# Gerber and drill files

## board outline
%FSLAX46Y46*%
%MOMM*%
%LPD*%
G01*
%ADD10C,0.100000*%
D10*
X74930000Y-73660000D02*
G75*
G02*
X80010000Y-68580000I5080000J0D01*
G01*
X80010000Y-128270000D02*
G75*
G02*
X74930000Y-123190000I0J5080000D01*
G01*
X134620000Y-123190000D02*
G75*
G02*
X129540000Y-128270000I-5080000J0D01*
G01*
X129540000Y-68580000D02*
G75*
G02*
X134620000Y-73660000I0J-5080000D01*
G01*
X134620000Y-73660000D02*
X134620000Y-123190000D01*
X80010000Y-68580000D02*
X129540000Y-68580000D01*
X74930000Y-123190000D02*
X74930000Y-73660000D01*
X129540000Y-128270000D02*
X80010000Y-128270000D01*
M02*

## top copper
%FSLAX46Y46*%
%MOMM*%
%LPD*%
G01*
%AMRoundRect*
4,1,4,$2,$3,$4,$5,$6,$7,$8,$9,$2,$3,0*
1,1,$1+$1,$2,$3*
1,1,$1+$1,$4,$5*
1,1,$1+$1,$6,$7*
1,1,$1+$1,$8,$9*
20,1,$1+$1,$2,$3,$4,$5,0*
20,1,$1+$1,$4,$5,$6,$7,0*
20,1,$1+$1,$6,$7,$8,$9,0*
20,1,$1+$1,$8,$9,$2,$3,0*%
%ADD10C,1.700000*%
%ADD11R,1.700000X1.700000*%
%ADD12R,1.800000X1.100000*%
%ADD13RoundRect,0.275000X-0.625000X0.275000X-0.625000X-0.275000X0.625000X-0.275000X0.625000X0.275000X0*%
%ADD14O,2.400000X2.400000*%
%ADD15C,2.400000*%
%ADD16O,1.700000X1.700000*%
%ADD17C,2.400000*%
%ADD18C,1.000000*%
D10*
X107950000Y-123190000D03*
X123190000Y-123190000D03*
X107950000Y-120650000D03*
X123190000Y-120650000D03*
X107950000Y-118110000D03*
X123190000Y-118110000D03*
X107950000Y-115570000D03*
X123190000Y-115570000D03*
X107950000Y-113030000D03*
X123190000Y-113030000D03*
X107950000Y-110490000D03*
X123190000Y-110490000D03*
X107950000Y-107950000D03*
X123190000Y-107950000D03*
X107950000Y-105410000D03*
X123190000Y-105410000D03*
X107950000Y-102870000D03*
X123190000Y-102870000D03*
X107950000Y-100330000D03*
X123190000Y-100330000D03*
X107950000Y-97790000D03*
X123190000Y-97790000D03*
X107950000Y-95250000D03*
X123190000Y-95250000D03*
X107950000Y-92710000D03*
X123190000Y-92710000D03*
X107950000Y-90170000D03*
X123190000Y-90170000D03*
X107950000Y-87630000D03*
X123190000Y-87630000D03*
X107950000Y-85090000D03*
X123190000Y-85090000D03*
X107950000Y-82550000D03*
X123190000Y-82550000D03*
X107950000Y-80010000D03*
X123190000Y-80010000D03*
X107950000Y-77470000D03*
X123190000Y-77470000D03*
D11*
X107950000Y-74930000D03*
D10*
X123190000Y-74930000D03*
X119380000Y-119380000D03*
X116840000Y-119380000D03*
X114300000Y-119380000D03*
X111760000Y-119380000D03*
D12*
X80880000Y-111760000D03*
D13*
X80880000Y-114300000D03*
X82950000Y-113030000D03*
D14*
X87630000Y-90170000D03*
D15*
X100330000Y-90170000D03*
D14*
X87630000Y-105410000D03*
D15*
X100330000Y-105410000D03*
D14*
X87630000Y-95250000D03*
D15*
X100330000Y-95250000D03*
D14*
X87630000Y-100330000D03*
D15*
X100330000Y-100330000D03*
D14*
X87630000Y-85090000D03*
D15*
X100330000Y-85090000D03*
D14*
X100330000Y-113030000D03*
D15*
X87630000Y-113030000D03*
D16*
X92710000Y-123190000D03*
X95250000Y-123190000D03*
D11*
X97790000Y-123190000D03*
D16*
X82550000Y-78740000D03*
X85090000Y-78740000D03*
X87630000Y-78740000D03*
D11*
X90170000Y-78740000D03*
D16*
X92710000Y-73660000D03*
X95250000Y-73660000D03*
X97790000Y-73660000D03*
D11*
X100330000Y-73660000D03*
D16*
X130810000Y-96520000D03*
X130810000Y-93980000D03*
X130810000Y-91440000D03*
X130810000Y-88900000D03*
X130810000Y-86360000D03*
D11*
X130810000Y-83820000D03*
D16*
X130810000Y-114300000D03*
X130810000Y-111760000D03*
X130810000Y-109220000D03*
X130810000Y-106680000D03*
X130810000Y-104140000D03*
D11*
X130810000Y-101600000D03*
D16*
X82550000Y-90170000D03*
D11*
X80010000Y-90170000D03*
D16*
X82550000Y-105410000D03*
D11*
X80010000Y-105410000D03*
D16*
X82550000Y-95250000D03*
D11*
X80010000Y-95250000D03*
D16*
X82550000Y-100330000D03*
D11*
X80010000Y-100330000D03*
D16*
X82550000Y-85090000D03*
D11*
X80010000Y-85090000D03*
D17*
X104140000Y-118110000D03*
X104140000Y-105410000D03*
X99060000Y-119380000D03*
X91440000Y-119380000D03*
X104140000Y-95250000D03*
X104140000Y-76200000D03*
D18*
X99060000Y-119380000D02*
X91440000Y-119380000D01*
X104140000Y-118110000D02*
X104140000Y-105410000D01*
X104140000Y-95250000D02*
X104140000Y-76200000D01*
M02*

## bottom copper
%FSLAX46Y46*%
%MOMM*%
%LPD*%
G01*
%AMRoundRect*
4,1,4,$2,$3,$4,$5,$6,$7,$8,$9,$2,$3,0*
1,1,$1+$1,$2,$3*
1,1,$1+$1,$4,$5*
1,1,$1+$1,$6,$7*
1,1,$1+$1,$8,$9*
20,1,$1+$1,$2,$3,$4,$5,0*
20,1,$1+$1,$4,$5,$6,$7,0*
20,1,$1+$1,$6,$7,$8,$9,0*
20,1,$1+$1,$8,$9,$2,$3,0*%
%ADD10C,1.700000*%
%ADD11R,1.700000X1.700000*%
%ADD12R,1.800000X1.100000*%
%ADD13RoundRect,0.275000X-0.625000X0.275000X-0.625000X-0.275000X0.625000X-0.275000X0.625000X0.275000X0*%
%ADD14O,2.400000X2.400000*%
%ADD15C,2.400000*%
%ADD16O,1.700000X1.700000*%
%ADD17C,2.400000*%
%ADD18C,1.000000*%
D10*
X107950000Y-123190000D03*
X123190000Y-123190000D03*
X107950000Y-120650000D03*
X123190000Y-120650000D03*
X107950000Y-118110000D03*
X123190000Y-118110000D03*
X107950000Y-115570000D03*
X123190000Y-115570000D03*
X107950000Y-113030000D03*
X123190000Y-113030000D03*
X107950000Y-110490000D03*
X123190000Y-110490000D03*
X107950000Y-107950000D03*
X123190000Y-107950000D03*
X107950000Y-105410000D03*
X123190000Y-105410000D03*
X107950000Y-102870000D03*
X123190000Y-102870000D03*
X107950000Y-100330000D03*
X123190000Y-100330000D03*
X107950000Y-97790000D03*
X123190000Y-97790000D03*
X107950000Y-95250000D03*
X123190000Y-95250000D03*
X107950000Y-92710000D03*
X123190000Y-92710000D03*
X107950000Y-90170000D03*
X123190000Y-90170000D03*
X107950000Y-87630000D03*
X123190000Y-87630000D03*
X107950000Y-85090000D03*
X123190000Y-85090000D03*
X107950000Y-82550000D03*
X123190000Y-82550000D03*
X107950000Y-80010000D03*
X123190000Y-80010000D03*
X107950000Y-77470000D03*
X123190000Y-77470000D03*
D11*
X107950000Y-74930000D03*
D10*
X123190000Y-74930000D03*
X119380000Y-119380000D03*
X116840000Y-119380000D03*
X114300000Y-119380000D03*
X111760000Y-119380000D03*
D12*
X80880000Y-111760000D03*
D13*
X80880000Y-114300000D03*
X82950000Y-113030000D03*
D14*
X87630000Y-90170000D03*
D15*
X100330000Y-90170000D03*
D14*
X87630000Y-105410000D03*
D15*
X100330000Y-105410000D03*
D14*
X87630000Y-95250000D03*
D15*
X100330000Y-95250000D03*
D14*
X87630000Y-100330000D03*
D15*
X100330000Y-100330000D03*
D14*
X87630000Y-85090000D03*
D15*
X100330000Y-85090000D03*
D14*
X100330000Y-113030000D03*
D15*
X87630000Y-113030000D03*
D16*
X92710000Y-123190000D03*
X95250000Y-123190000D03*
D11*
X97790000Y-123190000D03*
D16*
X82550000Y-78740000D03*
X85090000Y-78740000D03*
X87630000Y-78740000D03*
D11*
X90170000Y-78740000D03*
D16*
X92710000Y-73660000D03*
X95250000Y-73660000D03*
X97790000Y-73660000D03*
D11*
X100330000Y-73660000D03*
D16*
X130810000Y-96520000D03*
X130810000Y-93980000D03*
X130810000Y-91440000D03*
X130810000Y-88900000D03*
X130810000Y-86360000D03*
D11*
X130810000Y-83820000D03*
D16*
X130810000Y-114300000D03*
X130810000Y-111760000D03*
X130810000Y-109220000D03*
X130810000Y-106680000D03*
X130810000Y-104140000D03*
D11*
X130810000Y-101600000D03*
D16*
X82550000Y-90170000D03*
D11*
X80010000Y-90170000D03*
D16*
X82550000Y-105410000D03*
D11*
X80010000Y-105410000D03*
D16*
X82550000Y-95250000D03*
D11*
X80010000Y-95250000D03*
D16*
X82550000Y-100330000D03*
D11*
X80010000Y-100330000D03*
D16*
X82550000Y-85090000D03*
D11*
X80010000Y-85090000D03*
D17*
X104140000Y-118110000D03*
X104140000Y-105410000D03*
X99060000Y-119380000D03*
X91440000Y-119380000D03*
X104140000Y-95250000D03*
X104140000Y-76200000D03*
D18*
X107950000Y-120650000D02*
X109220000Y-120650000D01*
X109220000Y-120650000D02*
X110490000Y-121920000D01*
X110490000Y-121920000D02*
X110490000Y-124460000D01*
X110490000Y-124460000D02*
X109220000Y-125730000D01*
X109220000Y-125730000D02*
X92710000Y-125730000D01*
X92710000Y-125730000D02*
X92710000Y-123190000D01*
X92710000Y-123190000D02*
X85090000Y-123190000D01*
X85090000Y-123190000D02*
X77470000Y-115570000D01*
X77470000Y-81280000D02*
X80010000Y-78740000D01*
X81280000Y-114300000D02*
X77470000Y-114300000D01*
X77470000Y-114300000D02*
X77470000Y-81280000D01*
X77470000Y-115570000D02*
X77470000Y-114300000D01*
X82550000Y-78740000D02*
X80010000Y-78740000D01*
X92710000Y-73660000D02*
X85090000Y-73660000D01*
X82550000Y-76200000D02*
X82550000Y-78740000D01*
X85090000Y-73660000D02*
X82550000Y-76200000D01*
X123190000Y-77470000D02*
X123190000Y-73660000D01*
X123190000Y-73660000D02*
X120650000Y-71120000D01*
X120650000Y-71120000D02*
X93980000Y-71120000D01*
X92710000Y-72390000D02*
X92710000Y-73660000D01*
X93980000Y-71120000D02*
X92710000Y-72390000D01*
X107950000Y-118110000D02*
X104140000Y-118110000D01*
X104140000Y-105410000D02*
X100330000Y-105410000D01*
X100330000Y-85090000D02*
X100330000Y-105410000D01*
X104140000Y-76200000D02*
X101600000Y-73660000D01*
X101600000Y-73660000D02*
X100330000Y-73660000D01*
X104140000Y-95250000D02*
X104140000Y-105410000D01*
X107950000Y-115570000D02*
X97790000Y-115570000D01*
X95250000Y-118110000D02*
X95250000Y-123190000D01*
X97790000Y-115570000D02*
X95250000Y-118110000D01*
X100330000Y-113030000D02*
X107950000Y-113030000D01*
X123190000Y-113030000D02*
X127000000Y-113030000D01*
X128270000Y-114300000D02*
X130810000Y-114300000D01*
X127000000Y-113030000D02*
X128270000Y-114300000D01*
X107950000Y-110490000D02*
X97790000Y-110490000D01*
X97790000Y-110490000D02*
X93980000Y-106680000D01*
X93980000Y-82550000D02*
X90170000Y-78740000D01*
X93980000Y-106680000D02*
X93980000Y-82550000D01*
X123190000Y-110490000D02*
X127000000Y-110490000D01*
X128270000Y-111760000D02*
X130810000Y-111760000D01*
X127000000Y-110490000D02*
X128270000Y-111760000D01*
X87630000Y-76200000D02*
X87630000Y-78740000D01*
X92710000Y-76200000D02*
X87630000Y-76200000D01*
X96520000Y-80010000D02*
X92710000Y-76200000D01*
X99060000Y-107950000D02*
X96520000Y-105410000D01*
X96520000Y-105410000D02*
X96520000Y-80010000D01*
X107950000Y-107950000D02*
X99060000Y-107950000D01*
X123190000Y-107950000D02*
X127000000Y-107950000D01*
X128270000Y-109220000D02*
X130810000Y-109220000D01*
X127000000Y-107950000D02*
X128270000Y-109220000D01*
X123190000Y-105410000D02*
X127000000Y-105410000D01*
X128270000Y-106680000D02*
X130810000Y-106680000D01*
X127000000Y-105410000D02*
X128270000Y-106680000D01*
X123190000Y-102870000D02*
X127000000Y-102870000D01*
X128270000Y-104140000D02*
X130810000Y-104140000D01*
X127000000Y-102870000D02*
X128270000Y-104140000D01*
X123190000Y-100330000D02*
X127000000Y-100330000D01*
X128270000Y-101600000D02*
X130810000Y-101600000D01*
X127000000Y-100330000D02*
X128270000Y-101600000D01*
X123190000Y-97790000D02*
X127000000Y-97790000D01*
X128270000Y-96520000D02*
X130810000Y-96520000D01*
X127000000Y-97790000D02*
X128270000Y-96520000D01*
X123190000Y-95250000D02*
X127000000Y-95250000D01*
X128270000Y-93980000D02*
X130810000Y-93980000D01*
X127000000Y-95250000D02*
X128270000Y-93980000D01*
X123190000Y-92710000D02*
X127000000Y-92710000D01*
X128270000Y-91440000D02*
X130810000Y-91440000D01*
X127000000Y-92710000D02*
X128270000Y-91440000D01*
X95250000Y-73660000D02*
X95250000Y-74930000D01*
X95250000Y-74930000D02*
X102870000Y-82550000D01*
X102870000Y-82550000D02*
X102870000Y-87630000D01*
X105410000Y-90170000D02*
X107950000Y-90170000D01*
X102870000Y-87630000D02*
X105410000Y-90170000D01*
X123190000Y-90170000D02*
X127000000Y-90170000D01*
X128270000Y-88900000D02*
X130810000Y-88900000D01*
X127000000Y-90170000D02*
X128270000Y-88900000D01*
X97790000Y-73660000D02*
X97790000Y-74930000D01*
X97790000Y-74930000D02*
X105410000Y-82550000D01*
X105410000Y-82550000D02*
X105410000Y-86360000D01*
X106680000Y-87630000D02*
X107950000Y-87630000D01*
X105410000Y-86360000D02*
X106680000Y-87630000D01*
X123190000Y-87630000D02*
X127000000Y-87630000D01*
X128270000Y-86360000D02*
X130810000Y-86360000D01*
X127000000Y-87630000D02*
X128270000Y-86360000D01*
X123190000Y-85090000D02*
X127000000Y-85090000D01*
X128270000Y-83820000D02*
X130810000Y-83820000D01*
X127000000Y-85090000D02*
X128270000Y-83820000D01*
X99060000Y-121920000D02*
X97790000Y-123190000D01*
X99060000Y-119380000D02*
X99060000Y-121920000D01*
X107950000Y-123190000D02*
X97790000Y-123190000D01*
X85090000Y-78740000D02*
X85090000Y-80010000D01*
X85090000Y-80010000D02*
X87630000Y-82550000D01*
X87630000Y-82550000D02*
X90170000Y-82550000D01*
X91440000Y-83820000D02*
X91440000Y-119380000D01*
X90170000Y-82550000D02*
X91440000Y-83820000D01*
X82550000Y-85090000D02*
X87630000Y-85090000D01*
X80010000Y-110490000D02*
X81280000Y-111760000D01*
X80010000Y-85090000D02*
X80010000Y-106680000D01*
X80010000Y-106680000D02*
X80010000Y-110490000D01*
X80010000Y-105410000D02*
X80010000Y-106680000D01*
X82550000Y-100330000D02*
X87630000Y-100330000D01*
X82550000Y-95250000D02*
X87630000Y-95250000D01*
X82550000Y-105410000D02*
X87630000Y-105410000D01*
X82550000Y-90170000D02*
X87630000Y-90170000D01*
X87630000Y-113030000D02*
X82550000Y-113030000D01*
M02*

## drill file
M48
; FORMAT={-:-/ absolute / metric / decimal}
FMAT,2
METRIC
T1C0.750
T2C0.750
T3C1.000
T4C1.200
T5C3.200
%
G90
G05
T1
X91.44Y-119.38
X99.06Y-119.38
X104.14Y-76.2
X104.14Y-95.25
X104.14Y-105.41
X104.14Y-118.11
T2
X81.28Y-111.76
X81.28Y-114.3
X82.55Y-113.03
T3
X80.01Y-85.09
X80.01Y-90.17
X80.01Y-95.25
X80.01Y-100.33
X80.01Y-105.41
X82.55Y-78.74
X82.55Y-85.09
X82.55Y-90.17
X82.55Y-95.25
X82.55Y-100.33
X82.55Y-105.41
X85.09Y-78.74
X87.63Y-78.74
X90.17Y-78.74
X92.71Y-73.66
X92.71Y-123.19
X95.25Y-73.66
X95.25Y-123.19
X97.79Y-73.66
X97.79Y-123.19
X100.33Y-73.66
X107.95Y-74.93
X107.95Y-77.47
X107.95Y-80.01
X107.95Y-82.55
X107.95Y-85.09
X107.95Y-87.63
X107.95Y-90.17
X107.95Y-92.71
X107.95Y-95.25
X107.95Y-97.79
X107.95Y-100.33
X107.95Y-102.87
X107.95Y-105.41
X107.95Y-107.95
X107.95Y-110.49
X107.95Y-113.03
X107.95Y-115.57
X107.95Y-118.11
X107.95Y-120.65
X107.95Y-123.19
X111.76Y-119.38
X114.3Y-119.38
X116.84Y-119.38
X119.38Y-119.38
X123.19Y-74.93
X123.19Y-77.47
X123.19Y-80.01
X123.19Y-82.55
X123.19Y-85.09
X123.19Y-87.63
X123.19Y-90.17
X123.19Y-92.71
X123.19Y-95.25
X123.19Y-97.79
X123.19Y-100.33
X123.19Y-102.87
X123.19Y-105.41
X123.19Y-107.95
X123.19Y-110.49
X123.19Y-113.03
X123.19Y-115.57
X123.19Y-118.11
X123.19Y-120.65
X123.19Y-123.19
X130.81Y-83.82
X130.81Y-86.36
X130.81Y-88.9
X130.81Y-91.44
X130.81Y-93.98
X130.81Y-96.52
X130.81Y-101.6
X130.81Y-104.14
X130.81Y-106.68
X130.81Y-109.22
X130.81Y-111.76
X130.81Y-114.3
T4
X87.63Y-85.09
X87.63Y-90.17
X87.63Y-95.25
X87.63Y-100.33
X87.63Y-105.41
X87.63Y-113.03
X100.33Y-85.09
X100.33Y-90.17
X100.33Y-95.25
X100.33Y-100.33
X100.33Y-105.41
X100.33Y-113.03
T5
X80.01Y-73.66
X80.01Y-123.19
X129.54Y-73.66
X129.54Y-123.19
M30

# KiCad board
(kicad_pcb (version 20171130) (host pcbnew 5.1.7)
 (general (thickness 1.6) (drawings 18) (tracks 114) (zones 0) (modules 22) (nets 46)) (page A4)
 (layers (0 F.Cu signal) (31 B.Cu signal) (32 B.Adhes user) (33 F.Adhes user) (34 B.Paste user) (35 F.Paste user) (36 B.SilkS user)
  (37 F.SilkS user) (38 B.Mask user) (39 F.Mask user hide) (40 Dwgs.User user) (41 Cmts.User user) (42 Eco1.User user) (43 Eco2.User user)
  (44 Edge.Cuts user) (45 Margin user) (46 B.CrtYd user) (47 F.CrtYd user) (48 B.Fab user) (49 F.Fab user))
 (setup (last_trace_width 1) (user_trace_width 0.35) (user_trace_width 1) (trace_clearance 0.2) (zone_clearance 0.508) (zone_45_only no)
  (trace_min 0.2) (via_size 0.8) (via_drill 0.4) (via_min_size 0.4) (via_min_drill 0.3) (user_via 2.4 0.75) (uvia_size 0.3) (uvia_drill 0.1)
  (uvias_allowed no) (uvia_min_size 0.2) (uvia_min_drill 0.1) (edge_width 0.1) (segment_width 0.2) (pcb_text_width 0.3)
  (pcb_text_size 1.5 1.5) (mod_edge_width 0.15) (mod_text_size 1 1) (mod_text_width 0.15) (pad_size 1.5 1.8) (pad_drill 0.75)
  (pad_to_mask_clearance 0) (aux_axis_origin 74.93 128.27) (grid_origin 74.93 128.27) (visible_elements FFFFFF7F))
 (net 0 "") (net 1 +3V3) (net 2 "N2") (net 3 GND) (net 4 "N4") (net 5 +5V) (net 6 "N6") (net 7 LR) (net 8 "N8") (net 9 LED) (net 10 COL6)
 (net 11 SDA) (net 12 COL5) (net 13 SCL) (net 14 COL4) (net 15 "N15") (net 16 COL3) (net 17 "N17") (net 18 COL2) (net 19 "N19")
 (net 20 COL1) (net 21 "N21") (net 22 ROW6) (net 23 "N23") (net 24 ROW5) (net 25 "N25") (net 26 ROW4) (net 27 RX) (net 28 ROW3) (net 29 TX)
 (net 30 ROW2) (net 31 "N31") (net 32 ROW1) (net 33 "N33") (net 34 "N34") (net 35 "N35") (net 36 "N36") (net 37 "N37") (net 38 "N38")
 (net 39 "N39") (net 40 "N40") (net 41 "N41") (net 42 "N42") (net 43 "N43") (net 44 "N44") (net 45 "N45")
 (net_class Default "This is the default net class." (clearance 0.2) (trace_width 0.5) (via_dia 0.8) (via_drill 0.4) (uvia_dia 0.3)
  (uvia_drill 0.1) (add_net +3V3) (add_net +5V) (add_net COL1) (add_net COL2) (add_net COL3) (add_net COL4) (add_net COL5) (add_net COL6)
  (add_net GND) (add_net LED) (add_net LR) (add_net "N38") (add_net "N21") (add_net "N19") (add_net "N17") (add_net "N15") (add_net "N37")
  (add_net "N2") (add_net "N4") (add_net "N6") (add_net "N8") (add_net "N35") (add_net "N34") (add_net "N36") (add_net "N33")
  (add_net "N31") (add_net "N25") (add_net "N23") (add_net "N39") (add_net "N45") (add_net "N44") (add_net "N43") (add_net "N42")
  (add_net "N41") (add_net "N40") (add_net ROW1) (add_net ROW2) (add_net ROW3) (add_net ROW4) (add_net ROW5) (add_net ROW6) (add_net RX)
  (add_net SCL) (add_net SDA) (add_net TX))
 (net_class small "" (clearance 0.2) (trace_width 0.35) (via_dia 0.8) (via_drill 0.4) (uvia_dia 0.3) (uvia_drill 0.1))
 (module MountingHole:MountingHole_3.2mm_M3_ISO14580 (layer F.Cu) (at 80.01 123.19)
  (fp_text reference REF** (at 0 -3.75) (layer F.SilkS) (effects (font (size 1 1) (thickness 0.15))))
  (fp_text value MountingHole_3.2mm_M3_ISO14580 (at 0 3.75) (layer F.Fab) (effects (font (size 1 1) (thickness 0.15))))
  (pad 1 np_thru_hole circle (at 0 0) (size 3.2 3.2) (drill 3.2) (layers *.Cu *.Mask)))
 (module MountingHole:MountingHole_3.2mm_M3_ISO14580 (layer F.Cu) (at 129.54 123.19)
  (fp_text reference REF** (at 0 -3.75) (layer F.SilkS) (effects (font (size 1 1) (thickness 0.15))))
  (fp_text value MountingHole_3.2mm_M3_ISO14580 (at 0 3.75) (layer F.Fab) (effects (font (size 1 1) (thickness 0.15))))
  (pad 1 np_thru_hole circle (at 0 0) (size 3.2 3.2) (drill 3.2) (layers *.Cu *.Mask)))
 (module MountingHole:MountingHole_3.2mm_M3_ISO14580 (layer F.Cu) (at 129.54 73.66)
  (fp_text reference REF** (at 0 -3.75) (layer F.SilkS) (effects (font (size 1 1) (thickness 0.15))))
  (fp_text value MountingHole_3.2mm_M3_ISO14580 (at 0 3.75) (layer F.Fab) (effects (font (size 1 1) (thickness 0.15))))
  (pad 1 np_thru_hole circle (at 0 0) (size 3.2 3.2) (drill 3.2) (layers *.Cu *.Mask)))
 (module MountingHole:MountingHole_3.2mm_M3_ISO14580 (layer F.Cu) (at 80.01 73.66)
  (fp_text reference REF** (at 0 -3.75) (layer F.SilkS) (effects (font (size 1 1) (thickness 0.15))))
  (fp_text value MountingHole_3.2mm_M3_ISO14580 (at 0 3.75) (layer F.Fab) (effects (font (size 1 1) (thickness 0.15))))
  (pad 1 np_thru_hole circle (at 0 0) (size 3.2 3.2) (drill 3.2) (layers *.Cu *.Mask)))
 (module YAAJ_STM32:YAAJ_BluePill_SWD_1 (layer F.Cu) (at 107.95 74.93)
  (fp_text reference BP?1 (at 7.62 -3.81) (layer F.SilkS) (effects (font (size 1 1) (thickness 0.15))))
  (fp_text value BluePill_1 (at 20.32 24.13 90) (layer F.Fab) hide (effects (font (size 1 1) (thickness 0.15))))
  (pad 20 thru_hole circle (at 0 48.26) (size 1.7 1.7) (drill 1) (layers *.Cu *.Mask) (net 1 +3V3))
  (pad 21 thru_hole circle (at 15.24 48.26) (size 1.7 1.7) (drill 1) (layers *.Cu *.Mask) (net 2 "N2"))
  (pad 19 thru_hole circle (at 0 45.72) (size 1.7 1.7) (drill 1) (layers *.Cu *.Mask) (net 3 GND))
  (pad 22 thru_hole circle (at 15.24 45.72) (size 1.7 1.7) (drill 1) (layers *.Cu *.Mask) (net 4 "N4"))
  (pad 18 thru_hole circle (at 0 43.18) (size 1.7 1.7) (drill 1) (layers *.Cu *.Mask) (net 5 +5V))
  (pad 23 thru_hole circle (at 15.24 43.18) (size 1.7 1.7) (drill 1) (layers *.Cu *.Mask) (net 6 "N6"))
  (pad 17 thru_hole circle (at 0 40.64) (size 1.7 1.7) (drill 1) (layers *.Cu *.Mask) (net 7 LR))
  (pad 24 thru_hole circle (at 15.24 40.64) (size 1.7 1.7) (drill 1) (layers *.Cu *.Mask) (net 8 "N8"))
  (pad 16 thru_hole circle (at 0 38.1) (size 1.7 1.7) (drill 1) (layers *.Cu *.Mask) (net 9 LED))
  (pad 25 thru_hole circle (at 15.24 38.1) (size 1.7 1.7) (drill 1) (layers *.Cu *.Mask) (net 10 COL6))
  (pad 15 thru_hole circle (at 0 35.56) (size 1.7 1.7) (drill 1) (layers *.Cu *.Mask) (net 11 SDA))
  (pad 26 thru_hole circle (at 15.24 35.56) (size 1.7 1.7) (drill 1) (layers *.Cu *.Mask) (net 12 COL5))
  (pad 14 thru_hole circle (at 0 33.02) (size 1.7 1.7) (drill 1) (layers *.Cu *.Mask) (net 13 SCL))
  (pad 27 thru_hole circle (at 15.24 33.02) (size 1.7 1.7) (drill 1) (layers *.Cu *.Mask) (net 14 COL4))
  (pad 13 thru_hole circle (at 0 30.48) (size 1.7 1.7) (drill 1) (layers *.Cu *.Mask) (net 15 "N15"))
  (pad 28 thru_hole circle (at 15.24 30.48) (size 1.7 1.7) (drill 1) (layers *.Cu *.Mask) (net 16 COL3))
  (pad 12 thru_hole circle (at 0 27.94) (size 1.7 1.7) (drill 1) (layers *.Cu *.Mask) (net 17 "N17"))
  (pad 29 thru_hole circle (at 15.24 27.94) (size 1.7 1.7) (drill 1) (layers *.Cu *.Mask) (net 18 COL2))
  (pad 11 thru_hole circle (at 0 25.4) (size 1.7 1.7) (drill 1) (layers *.Cu *.Mask) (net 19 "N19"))
  (pad 30 thru_hole circle (at 15.24 25.4) (size 1.7 1.7) (drill 1) (layers *.Cu *.Mask) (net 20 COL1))
  (pad 10 thru_hole circle (at 0 22.86) (size 1.7 1.7) (drill 1) (layers *.Cu *.Mask) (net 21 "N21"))
  (pad 31 thru_hole circle (at 15.24 22.86) (size 1.7 1.7) (drill 1) (layers *.Cu *.Mask) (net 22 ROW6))
  (pad 9 thru_hole circle (at 0 20.32) (size 1.7 1.7) (drill 1) (layers *.Cu *.Mask) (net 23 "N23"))
  (pad 32 thru_hole circle (at 15.24 20.32) (size 1.7 1.7) (drill 1) (layers *.Cu *.Mask) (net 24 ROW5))
  (pad 8 thru_hole circle (at 0 17.78) (size 1.7 1.7) (drill 1) (layers *.Cu *.Mask) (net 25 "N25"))
  (pad 33 thru_hole circle (at 15.24 17.78) (size 1.7 1.7) (drill 1) (layers *.Cu *.Mask) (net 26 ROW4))
  (pad 7 thru_hole circle (at 0 15.24) (size 1.7 1.7) (drill 1) (layers *.Cu *.Mask) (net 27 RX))
  (pad 34 thru_hole circle (at 15.24 15.24) (size 1.7 1.7) (drill 1) (layers *.Cu *.Mask) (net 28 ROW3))
  (pad 6 thru_hole circle (at 0 12.7) (size 1.7 1.7) (drill 1) (layers *.Cu *.Mask) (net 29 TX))
  (pad 35 thru_hole circle (at 15.24 12.7) (size 1.7 1.7) (drill 1) (layers *.Cu *.Mask) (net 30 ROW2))
  (pad 5 thru_hole circle (at 0 10.16) (size 1.7 1.7) (drill 1) (layers *.Cu *.Mask) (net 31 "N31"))
  (pad 36 thru_hole circle (at 15.24 10.16) (size 1.7 1.7) (drill 1) (layers *.Cu *.Mask) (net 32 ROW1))
  (pad 4 thru_hole circle (at 0 7.62) (size 1.7 1.7) (drill 1) (layers *.Cu *.Mask) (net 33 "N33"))
  (pad 37 thru_hole circle (at 15.24 7.62) (size 1.7 1.7) (drill 1) (layers *.Cu *.Mask) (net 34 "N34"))
  (pad 3 thru_hole circle (at 0 5.08) (size 1.7 1.7) (drill 1) (layers *.Cu *.Mask) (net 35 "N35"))
  (pad 38 thru_hole circle (at 15.24 5.08) (size 1.7 1.7) (drill 1) (layers *.Cu *.Mask) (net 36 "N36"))
  (pad 2 thru_hole circle (at 0 2.54) (size 1.7 1.7) (drill 1) (layers *.Cu *.Mask) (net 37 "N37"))
  (pad 39 thru_hole circle (at 15.24 2.54) (size 1.7 1.7) (drill 1) (layers *.Cu *.Mask) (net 3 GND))
  (pad 1 thru_hole rect (at 0 0) (size 1.7 1.7) (drill 1) (layers *.Cu *.Mask) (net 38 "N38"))
  (pad 40 thru_hole circle (at 15.24 0) (size 1.7 1.7) (drill 1) (layers *.Cu *.Mask) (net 3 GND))
  (pad 41 thru_hole circle (at 11.43 44.45) (size 1.7 1.7) (drill 1) (layers *.Cu *.Mask))
  (pad 42 thru_hole circle (at 8.89 44.45) (size 1.7 1.7) (drill 1) (layers *.Cu *.Mask))
  (pad 43 thru_hole circle (at 6.35 44.45) (size 1.7 1.7) (drill 1) (layers *.Cu *.Mask))
  (pad 44 thru_hole circle (at 3.81 44.45) (size 1.7 1.7) (drill 1) (layers *.Cu *.Mask)))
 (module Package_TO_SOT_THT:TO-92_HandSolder (layer F.Cu) (at 81.28 111.76 270)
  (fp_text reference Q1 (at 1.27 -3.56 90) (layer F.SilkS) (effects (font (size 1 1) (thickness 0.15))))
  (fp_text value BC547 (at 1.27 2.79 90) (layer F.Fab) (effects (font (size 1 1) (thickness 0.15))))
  (pad 1 thru_hole rect (at 0 0 270) (size 1.1 1.8) (drill 0.75 (offset 0 0.4)) (layers *.Cu *.Mask) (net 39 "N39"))
  (pad 3 thru_hole roundrect (at 2.54 0 270) (size 1.1 1.8) (drill 0.75 (offset 0 0.4)) (layers *.Cu *.Mask) (roundrect_rratio 0.25)
   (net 3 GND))
  (pad 2 thru_hole roundrect (at 1.27 -1.27 270) (size 1.1 1.8) (drill 0.75 (offset 0 -0.4)) (layers *.Cu *.Mask) (roundrect_rratio 0.25)
   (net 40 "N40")))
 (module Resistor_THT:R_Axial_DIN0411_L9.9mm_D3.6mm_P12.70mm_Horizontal (layer F.Cu) (at 100.33 90.17 180)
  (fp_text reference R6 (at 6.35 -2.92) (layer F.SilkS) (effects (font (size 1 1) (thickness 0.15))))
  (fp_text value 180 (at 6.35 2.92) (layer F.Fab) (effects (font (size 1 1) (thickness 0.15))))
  (pad 2 thru_hole oval (at 12.7 0 180) (size 2.4 2.4) (drill 1.2) (layers *.Cu *.Mask) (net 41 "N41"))
  (pad 1 thru_hole circle (at 0 0 180) (size 2.4 2.4) (drill 1.2) (layers *.Cu *.Mask) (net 5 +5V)))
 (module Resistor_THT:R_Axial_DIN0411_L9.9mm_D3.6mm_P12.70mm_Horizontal (layer F.Cu) (at 100.33 105.41 180)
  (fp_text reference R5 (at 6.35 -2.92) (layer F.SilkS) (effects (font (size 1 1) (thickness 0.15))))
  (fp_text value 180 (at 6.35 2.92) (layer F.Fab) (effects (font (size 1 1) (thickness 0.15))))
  (pad 2 thru_hole oval (at 12.7 0 180) (size 2.4 2.4) (drill 1.2) (layers *.Cu *.Mask) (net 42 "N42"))
  (pad 1 thru_hole circle (at 0 0 180) (size 2.4 2.4) (drill 1.2) (layers *.Cu *.Mask) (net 5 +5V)))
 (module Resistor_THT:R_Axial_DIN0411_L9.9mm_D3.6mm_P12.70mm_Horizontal (layer F.Cu) (at 100.33 95.25 180)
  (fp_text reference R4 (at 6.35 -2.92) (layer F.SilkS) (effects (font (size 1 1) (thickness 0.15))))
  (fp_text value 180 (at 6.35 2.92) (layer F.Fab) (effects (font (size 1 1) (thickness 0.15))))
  (pad 2 thru_hole oval (at 12.7 0 180) (size 2.4 2.4) (drill 1.2) (layers *.Cu *.Mask) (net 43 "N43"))
  (pad 1 thru_hole circle (at 0 0 180) (size 2.4 2.4) (drill 1.2) (layers *.Cu *.Mask) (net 5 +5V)))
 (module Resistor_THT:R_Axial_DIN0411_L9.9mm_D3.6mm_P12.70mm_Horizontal (layer F.Cu) (at 100.33 100.33 180)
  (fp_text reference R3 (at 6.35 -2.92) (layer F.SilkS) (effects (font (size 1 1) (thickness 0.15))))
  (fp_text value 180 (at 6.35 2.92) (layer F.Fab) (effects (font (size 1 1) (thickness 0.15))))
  (pad 2 thru_hole oval (at 12.7 0 180) (size 2.4 2.4) (drill 1.2) (layers *.Cu *.Mask) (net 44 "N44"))
  (pad 1 thru_hole circle (at 0 0 180) (size 2.4 2.4) (drill 1.2) (layers *.Cu *.Mask) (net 5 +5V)))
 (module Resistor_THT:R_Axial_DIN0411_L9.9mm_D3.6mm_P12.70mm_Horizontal (layer F.Cu) (at 100.33 85.09 180)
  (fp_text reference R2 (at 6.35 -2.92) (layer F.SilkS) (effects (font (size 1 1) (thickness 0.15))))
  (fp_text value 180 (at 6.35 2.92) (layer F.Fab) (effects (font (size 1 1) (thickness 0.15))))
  (pad 2 thru_hole oval (at 12.7 0 180) (size 2.4 2.4) (drill 1.2) (layers *.Cu *.Mask) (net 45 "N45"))
  (pad 1 thru_hole circle (at 0 0 180) (size 2.4 2.4) (drill 1.2) (layers *.Cu *.Mask) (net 5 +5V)))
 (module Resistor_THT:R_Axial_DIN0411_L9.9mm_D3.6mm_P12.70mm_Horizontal (layer F.Cu) (at 87.63 113.03)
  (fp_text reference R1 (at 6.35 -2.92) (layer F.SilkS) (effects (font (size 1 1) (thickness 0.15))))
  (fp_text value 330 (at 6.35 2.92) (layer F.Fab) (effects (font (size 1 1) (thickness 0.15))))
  (pad 2 thru_hole oval (at 12.7 0) (size 2.4 2.4) (drill 1.2) (layers *.Cu *.Mask) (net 9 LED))
  (pad 1 thru_hole circle (at 0 0) (size 2.4 2.4) (drill 1.2) (layers *.Cu *.Mask) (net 40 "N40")))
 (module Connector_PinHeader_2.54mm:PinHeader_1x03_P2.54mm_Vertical (layer F.Cu) (at 97.79 123.19 270)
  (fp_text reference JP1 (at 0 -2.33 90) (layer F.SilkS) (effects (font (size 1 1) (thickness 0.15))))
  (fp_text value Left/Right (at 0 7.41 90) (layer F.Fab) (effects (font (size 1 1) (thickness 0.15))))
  (pad 3 thru_hole oval (at 0 5.08 270) (size 1.7 1.7) (drill 1) (layers *.Cu *.Mask) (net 3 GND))
  (pad 2 thru_hole oval (at 0 2.54 270) (size 1.7 1.7) (drill 1) (layers *.Cu *.Mask) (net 7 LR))
  (pad 1 thru_hole rect (at 0 0 270) (size 1.7 1.7) (drill 1) (layers *.Cu *.Mask) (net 1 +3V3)))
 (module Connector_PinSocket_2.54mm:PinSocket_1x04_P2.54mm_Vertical (layer F.Cu) (at 90.17 78.74 270)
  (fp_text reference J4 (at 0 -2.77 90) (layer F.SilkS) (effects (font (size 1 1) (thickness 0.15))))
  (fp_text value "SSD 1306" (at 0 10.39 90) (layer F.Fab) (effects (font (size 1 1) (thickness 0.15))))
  (pad 4 thru_hole oval (at 0 7.62 270) (size 1.7 1.7) (drill 1) (layers *.Cu *.Mask) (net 3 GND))
  (pad 3 thru_hole oval (at 0 5.08 270) (size 1.7 1.7) (drill 1) (layers *.Cu *.Mask) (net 1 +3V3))
  (pad 2 thru_hole oval (at 0 2.54 270) (size 1.7 1.7) (drill 1) (layers *.Cu *.Mask) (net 13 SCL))
  (pad 1 thru_hole rect (at 0 0 270) (size 1.7 1.7) (drill 1) (layers *.Cu *.Mask) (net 11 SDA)))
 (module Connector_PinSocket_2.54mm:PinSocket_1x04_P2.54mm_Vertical (layer F.Cu) (at 100.33 73.66 270)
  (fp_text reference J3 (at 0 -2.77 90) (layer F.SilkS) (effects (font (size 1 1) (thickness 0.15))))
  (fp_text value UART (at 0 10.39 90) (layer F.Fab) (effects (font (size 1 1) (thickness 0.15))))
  (pad 4 thru_hole oval (at 0 7.62 270) (size 1.7 1.7) (drill 1) (layers *.Cu *.Mask) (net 3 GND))
  (pad 3 thru_hole oval (at 0 5.08 270) (size 1.7 1.7) (drill 1) (layers *.Cu *.Mask) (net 27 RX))
  (pad 2 thru_hole oval (at 0 2.54 270) (size 1.7 1.7) (drill 1) (layers *.Cu *.Mask) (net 29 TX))
  (pad 1 thru_hole rect (at 0 0 270) (size 1.7 1.7) (drill 1) (layers *.Cu *.Mask) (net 5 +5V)))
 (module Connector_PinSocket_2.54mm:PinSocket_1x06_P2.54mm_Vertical (layer F.Cu) (at 130.81 83.82)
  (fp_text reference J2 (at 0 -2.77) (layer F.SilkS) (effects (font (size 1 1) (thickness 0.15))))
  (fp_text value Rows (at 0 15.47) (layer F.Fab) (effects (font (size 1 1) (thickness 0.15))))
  (pad 6 thru_hole oval (at 0 12.7) (size 1.7 1.7) (drill 1) (layers *.Cu *.Mask) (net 22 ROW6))
  (pad 5 thru_hole oval (at 0 10.16) (size 1.7 1.7) (drill 1) (layers *.Cu *.Mask) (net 24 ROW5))
  (pad 4 thru_hole oval (at 0 7.62) (size 1.7 1.7) (drill 1) (layers *.Cu *.Mask) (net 26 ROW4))
  (pad 3 thru_hole oval (at 0 5.08) (size 1.7 1.7) (drill 1) (layers *.Cu *.Mask) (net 28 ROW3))
  (pad 2 thru_hole oval (at 0 2.54) (size 1.7 1.7) (drill 1) (layers *.Cu *.Mask) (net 30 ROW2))
  (pad 1 thru_hole rect (at 0 0) (size 1.7 1.7) (drill 1) (layers *.Cu *.Mask) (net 32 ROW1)))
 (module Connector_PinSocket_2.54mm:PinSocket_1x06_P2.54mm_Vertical (layer F.Cu) (at 130.81 101.6)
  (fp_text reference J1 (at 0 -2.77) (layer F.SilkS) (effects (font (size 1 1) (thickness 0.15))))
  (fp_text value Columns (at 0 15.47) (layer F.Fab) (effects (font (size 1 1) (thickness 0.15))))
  (pad 6 thru_hole oval (at 0 12.7) (size 1.7 1.7) (drill 1) (layers *.Cu *.Mask) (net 10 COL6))
  (pad 5 thru_hole oval (at 0 10.16) (size 1.7 1.7) (drill 1) (layers *.Cu *.Mask) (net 12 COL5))
  (pad 4 thru_hole oval (at 0 7.62) (size 1.7 1.7) (drill 1) (layers *.Cu *.Mask) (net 14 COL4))
  (pad 3 thru_hole oval (at 0 5.08) (size 1.7 1.7) (drill 1) (layers *.Cu *.Mask) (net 16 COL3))
  (pad 2 thru_hole oval (at 0 2.54) (size 1.7 1.7) (drill 1) (layers *.Cu *.Mask) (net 18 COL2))
  (pad 1 thru_hole rect (at 0 0) (size 1.7 1.7) (drill 1) (layers *.Cu *.Mask) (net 20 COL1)))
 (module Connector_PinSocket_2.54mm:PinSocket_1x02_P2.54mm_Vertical (layer F.Cu) (at 80.01 90.17 90)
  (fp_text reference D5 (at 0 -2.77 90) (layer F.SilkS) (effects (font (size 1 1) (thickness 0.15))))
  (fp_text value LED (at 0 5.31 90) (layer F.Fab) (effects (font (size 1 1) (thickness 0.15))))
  (pad 2 thru_hole oval (at 0 2.54 90) (size 1.7 1.7) (drill 1) (layers *.Cu *.Mask) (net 41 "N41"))
  (pad 1 thru_hole rect (at 0 0 90) (size 1.7 1.7) (drill 1) (layers *.Cu *.Mask) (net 39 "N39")))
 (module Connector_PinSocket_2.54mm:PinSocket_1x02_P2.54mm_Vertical (layer F.Cu) (at 80.01 105.41 90)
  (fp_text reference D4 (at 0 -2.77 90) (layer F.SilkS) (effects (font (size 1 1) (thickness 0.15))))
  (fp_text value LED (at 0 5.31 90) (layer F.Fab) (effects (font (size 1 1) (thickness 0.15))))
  (pad 2 thru_hole oval (at 0 2.54 90) (size 1.7 1.7) (drill 1) (layers *.Cu *.Mask) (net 42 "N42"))
  (pad 1 thru_hole rect (at 0 0 90) (size 1.7 1.7) (drill 1) (layers *.Cu *.Mask) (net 39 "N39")))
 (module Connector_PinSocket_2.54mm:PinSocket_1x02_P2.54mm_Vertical (layer F.Cu) (at 80.01 95.25 90)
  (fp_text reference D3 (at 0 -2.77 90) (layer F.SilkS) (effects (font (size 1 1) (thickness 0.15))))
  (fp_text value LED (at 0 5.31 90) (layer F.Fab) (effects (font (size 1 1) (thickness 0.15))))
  (pad 2 thru_hole oval (at 0 2.54 90) (size 1.7 1.7) (drill 1) (layers *.Cu *.Mask) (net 43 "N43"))
  (pad 1 thru_hole rect (at 0 0 90) (size 1.7 1.7) (drill 1) (layers *.Cu *.Mask) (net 39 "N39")))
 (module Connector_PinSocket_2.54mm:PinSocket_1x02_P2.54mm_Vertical (layer F.Cu) (at 80.01 100.33 90)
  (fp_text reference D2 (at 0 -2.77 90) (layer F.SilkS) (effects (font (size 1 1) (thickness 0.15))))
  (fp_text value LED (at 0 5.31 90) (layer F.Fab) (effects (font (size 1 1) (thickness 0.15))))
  (pad 2 thru_hole oval (at 0 2.54 90) (size 1.7 1.7) (drill 1) (layers *.Cu *.Mask) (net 44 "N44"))
  (pad 1 thru_hole rect (at 0 0 90) (size 1.7 1.7) (drill 1) (layers *.Cu *.Mask) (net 39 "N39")))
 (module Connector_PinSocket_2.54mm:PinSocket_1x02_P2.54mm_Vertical (layer F.Cu) (at 80.01 85.09 90)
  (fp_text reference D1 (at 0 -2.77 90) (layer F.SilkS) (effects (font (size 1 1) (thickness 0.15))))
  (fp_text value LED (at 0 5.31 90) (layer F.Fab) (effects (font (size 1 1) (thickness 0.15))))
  (pad 2 thru_hole oval (at 0 2.54 90) (size 1.7 1.7) (drill 1) (layers *.Cu *.Mask) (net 45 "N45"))
  (pad 1 thru_hole rect (at 0 0 90) (size 1.7 1.7) (drill 1) (layers *.Cu *.Mask) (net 39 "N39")))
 (gr_arc (start 80.01 73.66) (end 80.01 68.58) (angle -90) (layer Edge.Cuts) (width 0.1))
 (gr_arc (start 80.01 123.19) (end 74.93 123.19) (angle -90) (layer Edge.Cuts) (width 0.1))
 (gr_arc (start 129.54 123.19) (end 129.54 128.27) (angle -90) (layer Edge.Cuts) (width 0.1))
 (gr_arc (start 129.54 73.66) (end 134.62 73.66) (angle -90) (layer Edge.Cuts) (width 0.1))
 (gr_line (start 134.62 73.66) (end 134.62 123.19) (layer Edge.Cuts) (width 0.1))
 (gr_line (start 80.01 68.58) (end 129.54 68.58) (layer Edge.Cuts) (width 0.1))
 (gr_line (start 74.93 123.19) (end 74.93 73.66) (layer Edge.Cuts) (width 0.1))
 (gr_line (start 129.54 128.27) (end 80.01 128.27) (layer Edge.Cuts) (width 0.1))
 (via (at 104.14 118.11) (size 2.4) (drill 0.75) (layers F.Cu B.Cu) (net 5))
 (via (at 104.14 105.41) (size 2.4) (drill 0.75) (layers F.Cu B.Cu) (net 5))
 (via (at 99.06 119.38) (size 2.4) (drill 0.75) (layers F.Cu B.Cu) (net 1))
 (via (at 91.44 119.38) (size 2.4) (drill 0.75) (layers F.Cu B.Cu) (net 1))
 (segment (start 99.06 119.38) (end 91.44 119.38) (width 1) (layer F.Cu) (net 1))
 (segment (start 104.14 118.11) (end 104.14 105.41) (width 1) (layer F.Cu) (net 5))
 (segment (start 107.95 120.65) (end 109.22 120.65) (width 1) (layer B.Cu) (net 3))
 (segment (start 109.22 120.65) (end 110.49 121.92) (width 1) (layer B.Cu) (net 3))
 (segment (start 110.49 121.92) (end 110.49 124.46) (width 1) (layer B.Cu) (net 3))
 (segment (start 110.49 124.46) (end 109.22 125.73) (width 1) (layer B.Cu) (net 3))
 (segment (start 109.22 125.73) (end 92.71 125.73) (width 1) (layer B.Cu) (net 3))
 (segment (start 92.71 125.73) (end 92.71 123.19) (width 1) (layer B.Cu) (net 3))
 (segment (start 92.71 123.19) (end 85.09 123.19) (width 1) (layer B.Cu) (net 3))
 (segment (start 85.09 123.19) (end 77.47 115.57) (width 1) (layer B.Cu) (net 3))
 (segment (start 77.47 81.28) (end 80.01 78.74) (width 1) (layer B.Cu) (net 3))
 (segment (start 81.28 114.3) (end 77.47 114.3) (width 1) (layer B.Cu) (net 3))
 (segment (start 77.47 114.3) (end 77.47 81.28) (width 1) (layer B.Cu) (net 3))
 (segment (start 77.47 115.57) (end 77.47 114.3) (width 1) (layer B.Cu) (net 3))
 (segment (start 82.55 78.74) (end 80.01 78.74) (width 1) (layer B.Cu) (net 3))
 (segment (start 92.71 73.66) (end 85.09 73.66) (width 1) (layer B.Cu) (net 3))
 (segment (start 82.55 76.2) (end 82.55 78.74) (width 1) (layer B.Cu) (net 3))
 (segment (start 85.09 73.66) (end 82.55 76.2) (width 1) (layer B.Cu) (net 3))
 (segment (start 123.19 77.47) (end 123.19 73.66) (width 1) (layer B.Cu) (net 3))
 (segment (start 123.19 73.66) (end 120.65 71.12) (width 1) (layer B.Cu) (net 3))
 (segment (start 120.65 71.12) (end 93.98 71.12) (width 1) (layer B.Cu) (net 3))
 (segment (start 92.71 72.39) (end 92.71 73.66) (width 1) (layer B.Cu) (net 3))
 (segment (start 93.98 71.12) (end 92.71 72.39) (width 1) (layer B.Cu) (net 3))
 (segment (start 107.95 118.11) (end 104.14 118.11) (width 1) (layer B.Cu) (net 5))
 (segment (start 104.14 105.41) (end 100.33 105.41) (width 1) (layer B.Cu) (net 5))
 (segment (start 100.33 85.09) (end 100.33 105.41) (width 1) (layer B.Cu) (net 5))
 (via (at 104.14 95.25) (size 2.4) (drill 0.75) (layers F.Cu B.Cu) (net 5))
 (via (at 104.14 76.2) (size 2.4) (drill 0.75) (layers F.Cu B.Cu) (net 5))
 (segment (start 104.14 95.25) (end 104.14 76.2) (width 1) (layer F.Cu) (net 5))
 (segment (start 104.14 76.2) (end 101.6 73.66) (width 1) (layer B.Cu) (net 5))
 (segment (start 101.6 73.66) (end 100.33 73.66) (width 1) (layer B.Cu) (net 5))
 (segment (start 104.14 95.25) (end 104.14 105.41) (width 1) (layer B.Cu) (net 5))
 (segment (start 107.95 115.57) (end 97.79 115.57) (width 1) (layer B.Cu) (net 7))
 (segment (start 95.25 118.11) (end 95.25 123.19) (width 1) (layer B.Cu) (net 7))
 (segment (start 97.79 115.57) (end 95.25 118.11) (width 1) (layer B.Cu) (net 7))
 (segment (start 100.33 113.03) (end 107.95 113.03) (width 1) (layer B.Cu) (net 9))
 (segment (start 123.19 113.03) (end 127 113.03) (width 1) (layer B.Cu) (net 10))
 (segment (start 128.27 114.3) (end 130.81 114.3) (width 1) (layer B.Cu) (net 10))
 (segment (start 127 113.03) (end 128.27 114.3) (width 1) (layer B.Cu) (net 10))
 (segment (start 107.95 110.49) (end 97.79 110.49) (width 1) (layer B.Cu) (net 11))
 (segment (start 97.79 110.49) (end 93.98 106.68) (width 1) (layer B.Cu) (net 11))
 (segment (start 93.98 82.55) (end 90.17 78.74) (width 1) (layer B.Cu) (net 11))
 (segment (start 93.98 106.68) (end 93.98 82.55) (width 1) (layer B.Cu) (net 11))
 (segment (start 123.19 110.49) (end 127 110.49) (width 1) (layer B.Cu) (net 12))
 (segment (start 128.27 111.76) (end 130.81 111.76) (width 1) (layer B.Cu) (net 12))
 (segment (start 127 110.49) (end 128.27 111.76) (width 1) (layer B.Cu) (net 12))
 (segment (start 87.63 76.2) (end 87.63 78.74) (width 1) (layer B.Cu) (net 13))
 (segment (start 92.71 76.2) (end 87.63 76.2) (width 1) (layer B.Cu) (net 13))
 (segment (start 96.52 80.01) (end 92.71 76.2) (width 1) (layer B.Cu) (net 13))
 (segment (start 99.06 107.95) (end 96.52 105.41) (width 1) (layer B.Cu) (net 13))
 (segment (start 96.52 105.41) (end 96.52 80.01) (width 1) (layer B.Cu) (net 13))
 (segment (start 107.95 107.95) (end 99.06 107.95) (width 1) (layer B.Cu) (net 13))
 (segment (start 123.19 107.95) (end 127 107.95) (width 1) (layer B.Cu) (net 14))
 (segment (start 128.27 109.22) (end 130.81 109.22) (width 1) (layer B.Cu) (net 14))
 (segment (start 127 107.95) (end 128.27 109.22) (width 1) (layer B.Cu) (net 14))
 (segment (start 123.19 105.41) (end 127 105.41) (width 1) (layer B.Cu) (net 16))
 (segment (start 128.27 106.68) (end 130.81 106.68) (width 1) (layer B.Cu) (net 16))
 (segment (start 127 105.41) (end 128.27 106.68) (width 1) (layer B.Cu) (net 16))
 (segment (start 123.19 102.87) (end 127 102.87) (width 1) (layer B.Cu) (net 18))
 (segment (start 128.27 104.14) (end 130.81 104.14) (width 1) (layer B.Cu) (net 18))
 (segment (start 127 102.87) (end 128.27 104.14) (width 1) (layer B.Cu) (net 18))
 (segment (start 123.19 100.33) (end 127 100.33) (width 1) (layer B.Cu) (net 20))
 (segment (start 128.27 101.6) (end 130.81 101.6) (width 1) (layer B.Cu) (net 20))
 (segment (start 127 100.33) (end 128.27 101.6) (width 1) (layer B.Cu) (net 20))
 (segment (start 123.19 97.79) (end 127 97.79) (width 1) (layer B.Cu) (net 22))
 (segment (start 128.27 96.52) (end 130.81 96.52) (width 1) (layer B.Cu) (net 22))
 (segment (start 127 97.79) (end 128.27 96.52) (width 1) (layer B.Cu) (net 22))
 (segment (start 123.19 95.25) (end 127 95.25) (width 1) (layer B.Cu) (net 24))
 (segment (start 128.27 93.98) (end 130.81 93.98) (width 1) (layer B.Cu) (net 24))
 (segment (start 127 95.25) (end 128.27 93.98) (width 1) (layer B.Cu) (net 24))
 (segment (start 123.19 92.71) (end 127 92.71) (width 1) (layer B.Cu) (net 26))
 (segment (start 128.27 91.44) (end 130.81 91.44) (width 1) (layer B.Cu) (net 26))
 (segment (start 127 92.71) (end 128.27 91.44) (width 1) (layer B.Cu) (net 26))
 (segment (start 95.25 73.66) (end 95.25 74.93) (width 1) (layer B.Cu) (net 27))
 (segment (start 95.25 74.93) (end 102.87 82.55) (width 1) (layer B.Cu) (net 27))
 (segment (start 102.87 82.55) (end 102.87 87.63) (width 1) (layer B.Cu) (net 27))
 (segment (start 105.41 90.17) (end 107.95 90.17) (width 1) (layer B.Cu) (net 27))
 (segment (start 102.87 87.63) (end 105.41 90.17) (width 1) (layer B.Cu) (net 27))
 (segment (start 123.19 90.17) (end 127 90.17) (width 1) (layer B.Cu) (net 28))
 (segment (start 128.27 88.9) (end 130.81 88.9) (width 1) (layer B.Cu) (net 28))
 (segment (start 127 90.17) (end 128.27 88.9) (width 1) (layer B.Cu) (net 28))
 (segment (start 97.79 73.66) (end 97.79 74.93) (width 1) (layer B.Cu) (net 29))
 (segment (start 97.79 74.93) (end 105.41 82.55) (width 1) (layer B.Cu) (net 29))
 (segment (start 105.41 82.55) (end 105.41 86.36) (width 1) (layer B.Cu) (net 29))
 (segment (start 106.68 87.63) (end 107.95 87.63) (width 1) (layer B.Cu) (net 29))
 (segment (start 105.41 86.36) (end 106.68 87.63) (width 1) (layer B.Cu) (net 29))
 (segment (start 123.19 87.63) (end 127 87.63) (width 1) (layer B.Cu) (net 30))
 (segment (start 128.27 86.36) (end 130.81 86.36) (width 1) (layer B.Cu) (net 30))
 (segment (start 127 87.63) (end 128.27 86.36) (width 1) (layer B.Cu) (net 30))
 (segment (start 123.19 85.09) (end 127 85.09) (width 1) (layer B.Cu) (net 32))
 (segment (start 128.27 83.82) (end 130.81 83.82) (width 1) (layer B.Cu) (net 32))
 (segment (start 127 85.09) (end 128.27 83.82) (width 1) (layer B.Cu) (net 32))
 (segment (start 99.06 121.92) (end 97.79 123.19) (width 1) (layer B.Cu) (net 1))
 (segment (start 99.06 119.38) (end 99.06 121.92) (width 1) (layer B.Cu) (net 1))
 (segment (start 107.95 123.19) (end 97.79 123.19) (width 1) (layer B.Cu) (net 1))
 (segment (start 85.09 78.74) (end 85.09 80.01) (width 1) (layer B.Cu) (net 1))
 (segment (start 85.09 80.01) (end 87.63 82.55) (width 1) (layer B.Cu) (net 1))
 (segment (start 87.63 82.55) (end 90.17 82.55) (width 1) (layer B.Cu) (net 1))
 (segment (start 91.44 83.82) (end 91.44 119.38) (width 1) (layer B.Cu) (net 1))
 (segment (start 90.17 82.55) (end 91.44 83.82) (width 1) (layer B.Cu) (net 1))
 (segment (start 82.55 85.09) (end 87.63 85.09) (width 1) (layer B.Cu) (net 45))
 (segment (start 80.01 110.49) (end 81.28 111.76) (width 1) (layer B.Cu) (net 39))
 (segment (start 80.01 85.09) (end 80.01 106.68) (width 1) (layer B.Cu) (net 39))
 (segment (start 80.01 106.68) (end 80.01 110.49) (width 1) (layer B.Cu) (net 39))
 (segment (start 80.01 105.41) (end 80.01 106.68) (width 1) (layer B.Cu) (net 39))
 (segment (start 82.55 100.33) (end 87.63 100.33) (width 1) (layer B.Cu) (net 44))
 (segment (start 82.55 95.25) (end 87.63 95.25) (width 1) (layer B.Cu) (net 43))
 (segment (start 82.55 105.41) (end 87.63 105.41) (width 1) (layer B.Cu) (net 42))
 (segment (start 82.55 90.17) (end 87.63 90.17) (width 1) (layer B.Cu) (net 41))
 (segment (start 87.63 113.03) (end 82.55 113.03) (width 1) (layer B.Cu) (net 40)))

